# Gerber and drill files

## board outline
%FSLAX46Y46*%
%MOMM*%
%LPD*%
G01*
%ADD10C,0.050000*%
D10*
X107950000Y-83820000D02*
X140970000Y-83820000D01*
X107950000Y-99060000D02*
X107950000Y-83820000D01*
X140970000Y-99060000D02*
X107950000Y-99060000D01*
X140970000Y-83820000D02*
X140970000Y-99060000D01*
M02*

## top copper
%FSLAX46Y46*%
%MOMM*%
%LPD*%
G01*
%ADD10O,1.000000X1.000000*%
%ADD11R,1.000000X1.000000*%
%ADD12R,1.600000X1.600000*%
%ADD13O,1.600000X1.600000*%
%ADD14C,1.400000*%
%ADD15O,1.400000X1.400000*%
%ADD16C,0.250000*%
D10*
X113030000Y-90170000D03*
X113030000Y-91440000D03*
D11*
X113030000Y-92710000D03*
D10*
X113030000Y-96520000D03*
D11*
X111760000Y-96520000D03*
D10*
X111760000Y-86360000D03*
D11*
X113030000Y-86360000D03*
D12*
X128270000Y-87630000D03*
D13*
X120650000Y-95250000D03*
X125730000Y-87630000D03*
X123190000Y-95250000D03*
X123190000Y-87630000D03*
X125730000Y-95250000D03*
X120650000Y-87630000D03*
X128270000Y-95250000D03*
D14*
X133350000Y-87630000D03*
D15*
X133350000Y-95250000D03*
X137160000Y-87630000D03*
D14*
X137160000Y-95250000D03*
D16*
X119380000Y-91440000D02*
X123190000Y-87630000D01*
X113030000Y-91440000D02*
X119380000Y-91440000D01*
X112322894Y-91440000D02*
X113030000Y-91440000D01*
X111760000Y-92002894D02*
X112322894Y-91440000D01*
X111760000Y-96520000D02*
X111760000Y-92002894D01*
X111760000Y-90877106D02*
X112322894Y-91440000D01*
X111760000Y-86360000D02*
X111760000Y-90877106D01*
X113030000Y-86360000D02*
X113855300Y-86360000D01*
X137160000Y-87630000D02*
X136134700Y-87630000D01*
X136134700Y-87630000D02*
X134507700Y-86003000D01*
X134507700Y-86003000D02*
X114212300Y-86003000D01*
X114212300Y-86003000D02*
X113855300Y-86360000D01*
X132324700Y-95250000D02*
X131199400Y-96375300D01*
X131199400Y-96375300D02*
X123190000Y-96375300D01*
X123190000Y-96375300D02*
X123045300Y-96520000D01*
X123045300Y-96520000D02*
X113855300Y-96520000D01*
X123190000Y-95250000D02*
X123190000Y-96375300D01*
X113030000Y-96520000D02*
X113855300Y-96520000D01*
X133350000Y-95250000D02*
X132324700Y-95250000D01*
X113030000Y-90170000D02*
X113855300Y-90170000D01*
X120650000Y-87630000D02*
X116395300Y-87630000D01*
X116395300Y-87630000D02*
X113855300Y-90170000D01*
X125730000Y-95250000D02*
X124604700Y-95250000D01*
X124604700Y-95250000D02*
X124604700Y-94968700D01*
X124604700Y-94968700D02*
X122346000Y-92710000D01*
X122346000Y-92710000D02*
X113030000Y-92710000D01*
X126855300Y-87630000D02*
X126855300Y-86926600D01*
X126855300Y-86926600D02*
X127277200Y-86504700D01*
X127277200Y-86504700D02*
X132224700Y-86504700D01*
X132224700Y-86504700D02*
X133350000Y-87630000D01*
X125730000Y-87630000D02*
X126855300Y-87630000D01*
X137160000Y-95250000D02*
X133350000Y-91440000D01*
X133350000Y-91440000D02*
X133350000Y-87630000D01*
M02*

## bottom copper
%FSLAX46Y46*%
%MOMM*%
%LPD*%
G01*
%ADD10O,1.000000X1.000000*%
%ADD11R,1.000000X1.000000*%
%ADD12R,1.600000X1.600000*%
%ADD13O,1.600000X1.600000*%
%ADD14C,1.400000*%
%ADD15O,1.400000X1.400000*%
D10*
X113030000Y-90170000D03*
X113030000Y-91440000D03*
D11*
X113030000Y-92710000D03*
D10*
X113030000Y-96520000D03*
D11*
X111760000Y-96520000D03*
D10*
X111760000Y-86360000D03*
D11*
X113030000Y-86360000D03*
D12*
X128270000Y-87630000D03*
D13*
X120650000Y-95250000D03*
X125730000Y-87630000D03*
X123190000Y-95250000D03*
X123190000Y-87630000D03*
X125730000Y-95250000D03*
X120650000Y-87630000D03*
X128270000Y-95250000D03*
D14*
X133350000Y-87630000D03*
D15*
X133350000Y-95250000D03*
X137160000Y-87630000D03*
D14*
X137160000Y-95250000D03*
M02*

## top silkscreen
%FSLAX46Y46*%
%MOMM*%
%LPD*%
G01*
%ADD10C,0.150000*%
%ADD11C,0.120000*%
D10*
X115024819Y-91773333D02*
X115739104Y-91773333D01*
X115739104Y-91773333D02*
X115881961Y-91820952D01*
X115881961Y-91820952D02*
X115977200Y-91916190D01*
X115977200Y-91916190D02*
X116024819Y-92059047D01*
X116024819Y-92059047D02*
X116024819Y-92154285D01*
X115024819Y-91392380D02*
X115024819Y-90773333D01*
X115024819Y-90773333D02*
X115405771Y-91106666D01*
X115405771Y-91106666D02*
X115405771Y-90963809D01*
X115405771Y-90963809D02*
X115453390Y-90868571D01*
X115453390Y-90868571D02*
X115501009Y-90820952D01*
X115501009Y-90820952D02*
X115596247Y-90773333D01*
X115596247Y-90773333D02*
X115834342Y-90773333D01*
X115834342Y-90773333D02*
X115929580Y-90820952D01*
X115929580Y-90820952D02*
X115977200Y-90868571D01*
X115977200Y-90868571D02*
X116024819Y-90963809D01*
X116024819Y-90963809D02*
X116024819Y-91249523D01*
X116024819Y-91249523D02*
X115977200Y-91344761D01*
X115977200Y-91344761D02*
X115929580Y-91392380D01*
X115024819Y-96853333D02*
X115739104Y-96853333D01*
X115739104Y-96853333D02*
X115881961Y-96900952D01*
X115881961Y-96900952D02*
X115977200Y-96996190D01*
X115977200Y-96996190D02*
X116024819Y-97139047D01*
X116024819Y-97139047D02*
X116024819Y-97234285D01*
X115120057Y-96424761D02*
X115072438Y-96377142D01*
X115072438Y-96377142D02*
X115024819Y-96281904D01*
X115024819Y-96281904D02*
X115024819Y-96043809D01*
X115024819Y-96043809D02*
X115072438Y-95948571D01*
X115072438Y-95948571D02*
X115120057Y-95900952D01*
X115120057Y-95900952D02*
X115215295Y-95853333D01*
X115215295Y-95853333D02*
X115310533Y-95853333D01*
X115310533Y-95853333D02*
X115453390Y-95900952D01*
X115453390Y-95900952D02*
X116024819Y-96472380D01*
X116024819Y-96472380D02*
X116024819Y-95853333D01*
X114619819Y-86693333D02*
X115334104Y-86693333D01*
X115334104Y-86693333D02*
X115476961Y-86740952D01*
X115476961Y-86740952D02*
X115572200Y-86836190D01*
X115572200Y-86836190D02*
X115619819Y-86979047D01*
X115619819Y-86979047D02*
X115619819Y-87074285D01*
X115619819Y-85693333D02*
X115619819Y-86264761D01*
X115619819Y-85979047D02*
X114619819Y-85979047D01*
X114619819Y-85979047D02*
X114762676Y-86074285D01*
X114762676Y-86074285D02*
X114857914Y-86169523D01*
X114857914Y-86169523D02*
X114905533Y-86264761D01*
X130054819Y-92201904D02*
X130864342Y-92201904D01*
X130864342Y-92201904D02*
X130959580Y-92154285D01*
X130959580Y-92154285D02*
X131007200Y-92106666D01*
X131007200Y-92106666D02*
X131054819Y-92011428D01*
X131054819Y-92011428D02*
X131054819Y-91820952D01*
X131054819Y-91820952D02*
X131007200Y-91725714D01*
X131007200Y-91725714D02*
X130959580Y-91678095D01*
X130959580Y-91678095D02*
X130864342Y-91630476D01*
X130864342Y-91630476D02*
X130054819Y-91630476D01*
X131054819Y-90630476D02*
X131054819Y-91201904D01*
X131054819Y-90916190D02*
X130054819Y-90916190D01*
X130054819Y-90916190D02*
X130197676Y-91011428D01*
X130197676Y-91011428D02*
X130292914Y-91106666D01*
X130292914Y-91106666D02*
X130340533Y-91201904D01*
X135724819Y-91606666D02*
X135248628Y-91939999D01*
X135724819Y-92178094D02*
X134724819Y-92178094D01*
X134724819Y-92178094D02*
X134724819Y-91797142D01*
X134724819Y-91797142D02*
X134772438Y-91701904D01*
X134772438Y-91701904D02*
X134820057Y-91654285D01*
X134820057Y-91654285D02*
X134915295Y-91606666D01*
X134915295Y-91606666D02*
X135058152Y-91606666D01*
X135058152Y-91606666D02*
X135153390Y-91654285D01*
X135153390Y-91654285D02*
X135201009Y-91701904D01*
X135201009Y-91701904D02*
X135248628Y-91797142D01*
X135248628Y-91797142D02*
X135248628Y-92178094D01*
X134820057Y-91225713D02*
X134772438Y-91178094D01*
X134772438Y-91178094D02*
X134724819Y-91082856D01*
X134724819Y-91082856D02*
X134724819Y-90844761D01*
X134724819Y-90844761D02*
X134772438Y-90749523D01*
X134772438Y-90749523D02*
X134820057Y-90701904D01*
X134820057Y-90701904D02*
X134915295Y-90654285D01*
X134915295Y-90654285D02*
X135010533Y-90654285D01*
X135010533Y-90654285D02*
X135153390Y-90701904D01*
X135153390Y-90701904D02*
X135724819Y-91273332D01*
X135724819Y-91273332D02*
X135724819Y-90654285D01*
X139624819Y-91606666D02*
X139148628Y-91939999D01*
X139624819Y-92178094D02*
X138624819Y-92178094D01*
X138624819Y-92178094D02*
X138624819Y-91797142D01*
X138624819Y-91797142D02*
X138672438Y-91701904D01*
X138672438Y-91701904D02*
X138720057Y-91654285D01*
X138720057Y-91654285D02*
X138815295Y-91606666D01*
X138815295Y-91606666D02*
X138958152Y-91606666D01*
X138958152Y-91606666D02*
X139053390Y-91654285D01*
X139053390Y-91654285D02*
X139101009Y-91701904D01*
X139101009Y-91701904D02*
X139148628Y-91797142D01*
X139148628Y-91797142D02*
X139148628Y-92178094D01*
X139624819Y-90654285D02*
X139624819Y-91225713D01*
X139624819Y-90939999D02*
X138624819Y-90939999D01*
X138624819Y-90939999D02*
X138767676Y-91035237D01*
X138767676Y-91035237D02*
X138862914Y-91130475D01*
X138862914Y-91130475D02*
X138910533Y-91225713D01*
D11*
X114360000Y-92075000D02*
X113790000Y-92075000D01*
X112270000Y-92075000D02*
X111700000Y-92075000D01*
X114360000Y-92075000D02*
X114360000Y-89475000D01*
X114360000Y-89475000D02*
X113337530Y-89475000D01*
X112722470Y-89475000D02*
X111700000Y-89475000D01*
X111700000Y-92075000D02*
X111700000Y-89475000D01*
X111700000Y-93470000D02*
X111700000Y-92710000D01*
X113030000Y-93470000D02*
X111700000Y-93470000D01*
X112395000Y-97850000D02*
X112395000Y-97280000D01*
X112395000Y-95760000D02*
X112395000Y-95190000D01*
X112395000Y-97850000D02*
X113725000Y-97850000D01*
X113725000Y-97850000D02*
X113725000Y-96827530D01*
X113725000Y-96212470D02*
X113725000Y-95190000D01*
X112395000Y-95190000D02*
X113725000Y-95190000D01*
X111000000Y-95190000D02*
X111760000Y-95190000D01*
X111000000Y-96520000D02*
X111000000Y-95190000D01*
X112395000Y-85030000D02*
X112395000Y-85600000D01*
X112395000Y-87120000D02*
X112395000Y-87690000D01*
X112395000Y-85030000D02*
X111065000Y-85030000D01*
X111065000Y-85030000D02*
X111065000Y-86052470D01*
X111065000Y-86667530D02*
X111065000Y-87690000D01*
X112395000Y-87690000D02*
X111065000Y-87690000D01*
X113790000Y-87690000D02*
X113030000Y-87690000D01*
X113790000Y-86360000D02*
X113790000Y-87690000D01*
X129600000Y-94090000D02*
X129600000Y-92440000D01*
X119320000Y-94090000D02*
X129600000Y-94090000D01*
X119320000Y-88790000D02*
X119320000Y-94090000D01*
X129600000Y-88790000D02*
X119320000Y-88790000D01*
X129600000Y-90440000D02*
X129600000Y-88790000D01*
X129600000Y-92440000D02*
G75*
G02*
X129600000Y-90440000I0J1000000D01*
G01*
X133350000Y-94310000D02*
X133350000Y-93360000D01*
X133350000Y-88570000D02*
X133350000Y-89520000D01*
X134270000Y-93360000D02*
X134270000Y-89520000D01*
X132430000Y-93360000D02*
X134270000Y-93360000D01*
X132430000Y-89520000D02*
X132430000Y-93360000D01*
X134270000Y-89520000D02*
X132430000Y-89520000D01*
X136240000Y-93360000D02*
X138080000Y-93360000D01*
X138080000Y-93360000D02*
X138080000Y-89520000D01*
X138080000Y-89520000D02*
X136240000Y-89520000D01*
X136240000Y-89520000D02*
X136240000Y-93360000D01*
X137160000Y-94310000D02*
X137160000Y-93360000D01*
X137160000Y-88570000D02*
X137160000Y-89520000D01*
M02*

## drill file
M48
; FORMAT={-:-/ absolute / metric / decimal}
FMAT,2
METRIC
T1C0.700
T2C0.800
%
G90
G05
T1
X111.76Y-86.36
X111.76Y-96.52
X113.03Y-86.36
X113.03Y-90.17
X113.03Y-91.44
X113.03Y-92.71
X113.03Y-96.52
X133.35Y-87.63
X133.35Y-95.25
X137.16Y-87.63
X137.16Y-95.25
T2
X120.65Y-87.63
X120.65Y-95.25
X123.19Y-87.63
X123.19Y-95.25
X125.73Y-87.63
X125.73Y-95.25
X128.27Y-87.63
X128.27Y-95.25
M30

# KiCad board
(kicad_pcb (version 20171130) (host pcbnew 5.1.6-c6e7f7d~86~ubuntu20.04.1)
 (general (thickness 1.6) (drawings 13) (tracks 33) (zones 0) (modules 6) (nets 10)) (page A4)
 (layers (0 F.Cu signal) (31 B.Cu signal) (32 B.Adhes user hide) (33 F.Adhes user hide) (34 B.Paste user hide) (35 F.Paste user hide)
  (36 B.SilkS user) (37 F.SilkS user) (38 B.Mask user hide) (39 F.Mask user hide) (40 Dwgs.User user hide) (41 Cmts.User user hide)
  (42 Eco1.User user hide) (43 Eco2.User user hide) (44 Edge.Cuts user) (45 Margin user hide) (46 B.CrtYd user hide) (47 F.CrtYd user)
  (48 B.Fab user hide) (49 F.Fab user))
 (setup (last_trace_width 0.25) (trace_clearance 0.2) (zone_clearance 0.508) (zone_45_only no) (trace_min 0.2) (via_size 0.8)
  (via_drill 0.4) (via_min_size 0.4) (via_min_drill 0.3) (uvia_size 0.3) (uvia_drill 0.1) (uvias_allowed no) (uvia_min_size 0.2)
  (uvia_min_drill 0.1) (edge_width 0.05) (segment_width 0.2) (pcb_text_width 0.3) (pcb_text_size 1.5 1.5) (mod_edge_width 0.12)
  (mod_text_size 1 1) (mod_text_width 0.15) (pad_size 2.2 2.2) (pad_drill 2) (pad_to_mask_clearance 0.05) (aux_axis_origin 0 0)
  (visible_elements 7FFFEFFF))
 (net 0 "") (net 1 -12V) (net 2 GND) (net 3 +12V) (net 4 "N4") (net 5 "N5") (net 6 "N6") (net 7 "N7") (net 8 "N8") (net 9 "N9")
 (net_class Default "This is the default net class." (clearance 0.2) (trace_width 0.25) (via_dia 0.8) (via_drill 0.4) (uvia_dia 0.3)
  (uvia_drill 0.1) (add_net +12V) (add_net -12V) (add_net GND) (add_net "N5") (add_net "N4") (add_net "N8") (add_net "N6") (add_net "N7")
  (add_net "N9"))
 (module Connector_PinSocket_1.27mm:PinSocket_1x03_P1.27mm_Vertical (layer F.Cu) (at 113.03 92.71 180)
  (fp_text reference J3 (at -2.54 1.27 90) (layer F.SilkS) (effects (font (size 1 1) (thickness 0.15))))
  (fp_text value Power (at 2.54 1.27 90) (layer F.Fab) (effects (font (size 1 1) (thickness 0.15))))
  (fp_line (start -1.33 0.635) (end -0.76 0.635) (layer F.SilkS) (width 0.12))
  (fp_line (start 0.76 0.635) (end 1.33 0.635) (layer F.SilkS) (width 0.12))
  (fp_line (start -1.33 0.635) (end -1.33 3.235) (layer F.SilkS) (width 0.12))
  (fp_line (start -1.33 3.235) (end -0.30753 3.235) (layer F.SilkS) (width 0.12))
  (fp_line (start 0.30753 3.235) (end 1.33 3.235) (layer F.SilkS) (width 0.12))
  (fp_line (start 1.33 0.635) (end 1.33 3.235) (layer F.SilkS) (width 0.12))
  (fp_line (start 1.33 -0.76) (end 1.33 0) (layer F.SilkS) (width 0.12))
  (fp_line (start 0 -0.76) (end 1.33 -0.76) (layer F.SilkS) (width 0.12))
  (pad 3 thru_hole oval (at 0 2.54 180) (size 1 1) (drill 0.7) (layers *.Cu *.Mask) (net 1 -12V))
  (pad 2 thru_hole oval (at 0 1.27 180) (size 1 1) (drill 0.7) (layers *.Cu *.Mask) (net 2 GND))
  (pad 1 thru_hole rect (at 0 0 180) (size 1 1) (drill 0.7) (layers *.Cu *.Mask) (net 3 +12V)))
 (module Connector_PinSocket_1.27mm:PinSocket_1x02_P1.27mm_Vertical (layer F.Cu) (at 111.76 96.52 90)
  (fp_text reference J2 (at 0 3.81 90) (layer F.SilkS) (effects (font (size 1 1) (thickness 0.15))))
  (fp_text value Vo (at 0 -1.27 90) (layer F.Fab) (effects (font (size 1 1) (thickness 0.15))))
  (fp_line (start -1.33 0.635) (end -0.76 0.635) (layer F.SilkS) (width 0.12))
  (fp_line (start 0.76 0.635) (end 1.33 0.635) (layer F.SilkS) (width 0.12))
  (fp_line (start -1.33 0.635) (end -1.33 1.965) (layer F.SilkS) (width 0.12))
  (fp_line (start -1.33 1.965) (end -0.30753 1.965) (layer F.SilkS) (width 0.12))
  (fp_line (start 0.30753 1.965) (end 1.33 1.965) (layer F.SilkS) (width 0.12))
  (fp_line (start 1.33 0.635) (end 1.33 1.965) (layer F.SilkS) (width 0.12))
  (fp_line (start 1.33 -0.76) (end 1.33 0) (layer F.SilkS) (width 0.12))
  (fp_line (start 0 -0.76) (end 1.33 -0.76) (layer F.SilkS) (width 0.12))
  (pad 2 thru_hole oval (at 0 1.27 90) (size 1 1) (drill 0.7) (layers *.Cu *.Mask) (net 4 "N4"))
  (pad 1 thru_hole rect (at 0 0 90) (size 1 1) (drill 0.7) (layers *.Cu *.Mask) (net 2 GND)))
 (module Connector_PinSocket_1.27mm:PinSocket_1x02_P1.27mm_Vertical (layer F.Cu) (at 113.03 86.36 270)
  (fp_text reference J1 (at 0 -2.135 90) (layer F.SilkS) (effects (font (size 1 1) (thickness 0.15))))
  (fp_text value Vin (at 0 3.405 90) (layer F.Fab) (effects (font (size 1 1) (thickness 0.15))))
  (fp_line (start -1.33 0.635) (end -0.76 0.635) (layer F.SilkS) (width 0.12))
  (fp_line (start 0.76 0.635) (end 1.33 0.635) (layer F.SilkS) (width 0.12))
  (fp_line (start -1.33 0.635) (end -1.33 1.965) (layer F.SilkS) (width 0.12))
  (fp_line (start -1.33 1.965) (end -0.30753 1.965) (layer F.SilkS) (width 0.12))
  (fp_line (start 0.30753 1.965) (end 1.33 1.965) (layer F.SilkS) (width 0.12))
  (fp_line (start 1.33 0.635) (end 1.33 1.965) (layer F.SilkS) (width 0.12))
  (fp_line (start 1.33 -0.76) (end 1.33 0) (layer F.SilkS) (width 0.12))
  (fp_line (start 0 -0.76) (end 1.33 -0.76) (layer F.SilkS) (width 0.12))
  (pad 2 thru_hole oval (at 0 1.27 270) (size 1 1) (drill 0.7) (layers *.Cu *.Mask) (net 2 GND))
  (pad 1 thru_hole rect (at 0 0 270) (size 1 1) (drill 0.7) (layers *.Cu *.Mask) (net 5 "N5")))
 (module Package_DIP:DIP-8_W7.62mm (layer F.Cu) (at 128.27 87.63 270)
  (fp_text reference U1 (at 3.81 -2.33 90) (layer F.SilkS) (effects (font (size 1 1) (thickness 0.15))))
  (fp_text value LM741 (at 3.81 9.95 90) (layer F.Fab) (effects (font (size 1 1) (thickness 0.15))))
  (fp_line (start 6.46 -1.33) (end 4.81 -1.33) (layer F.SilkS) (width 0.12))
  (fp_line (start 6.46 8.95) (end 6.46 -1.33) (layer F.SilkS) (width 0.12))
  (fp_line (start 1.16 8.95) (end 6.46 8.95) (layer F.SilkS) (width 0.12))
  (fp_line (start 1.16 -1.33) (end 1.16 8.95) (layer F.SilkS) (width 0.12))
  (fp_line (start 2.81 -1.33) (end 1.16 -1.33) (layer F.SilkS) (width 0.12))
  (fp_arc (start 3.81 -1.33) (end 2.81 -1.33) (angle -180) (layer F.SilkS) (width 0.12))
  (pad 1 thru_hole rect (at 0 0 270) (size 1.6 1.6) (drill 0.8) (layers *.Cu *.Mask) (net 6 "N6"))
  (pad 5 thru_hole oval (at 7.62 7.62 270) (size 1.6 1.6) (drill 0.8) (layers *.Cu *.Mask) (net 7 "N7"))
  (pad 2 thru_hole oval (at 0 2.54 270) (size 1.6 1.6) (drill 0.8) (layers *.Cu *.Mask) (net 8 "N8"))
  (pad 6 thru_hole oval (at 7.62 5.08 270) (size 1.6 1.6) (drill 0.8) (layers *.Cu *.Mask) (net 4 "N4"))
  (pad 3 thru_hole oval (at 0 5.08 270) (size 1.6 1.6) (drill 0.8) (layers *.Cu *.Mask) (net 2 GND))
  (pad 7 thru_hole oval (at 7.62 2.54 270) (size 1.6 1.6) (drill 0.8) (layers *.Cu *.Mask) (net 3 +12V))
  (pad 4 thru_hole oval (at 0 7.62 270) (size 1.6 1.6) (drill 0.8) (layers *.Cu *.Mask) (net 1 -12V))
  (pad 8 thru_hole oval (at 7.62 0 270) (size 1.6 1.6) (drill 0.8) (layers *.Cu *.Mask) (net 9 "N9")))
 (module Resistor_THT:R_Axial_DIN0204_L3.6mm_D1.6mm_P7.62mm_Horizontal (layer F.Cu) (at 133.35 87.63 270)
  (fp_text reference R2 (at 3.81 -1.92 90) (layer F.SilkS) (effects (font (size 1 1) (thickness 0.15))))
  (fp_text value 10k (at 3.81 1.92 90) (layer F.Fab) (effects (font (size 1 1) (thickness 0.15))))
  (fp_line (start 6.68 0) (end 5.73 0) (layer F.SilkS) (width 0.12))
  (fp_line (start 0.94 0) (end 1.89 0) (layer F.SilkS) (width 0.12))
  (fp_line (start 5.73 -0.92) (end 1.89 -0.92) (layer F.SilkS) (width 0.12))
  (fp_line (start 5.73 0.92) (end 5.73 -0.92) (layer F.SilkS) (width 0.12))
  (fp_line (start 1.89 0.92) (end 5.73 0.92) (layer F.SilkS) (width 0.12))
  (fp_line (start 1.89 -0.92) (end 1.89 0.92) (layer F.SilkS) (width 0.12))
  (pad 1 thru_hole circle (at 0 0 270) (size 1.4 1.4) (drill 0.7) (layers *.Cu *.Mask) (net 8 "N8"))
  (pad 2 thru_hole oval (at 7.62 0 270) (size 1.4 1.4) (drill 0.7) (layers *.Cu *.Mask) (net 4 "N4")))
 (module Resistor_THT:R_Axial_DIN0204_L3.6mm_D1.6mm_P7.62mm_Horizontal (layer F.Cu) (at 137.16 95.25 90)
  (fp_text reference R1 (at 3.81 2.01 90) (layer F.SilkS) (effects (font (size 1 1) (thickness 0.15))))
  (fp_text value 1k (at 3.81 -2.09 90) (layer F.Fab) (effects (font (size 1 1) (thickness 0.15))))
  (fp_line (start 1.89 -0.92) (end 1.89 0.92) (layer F.SilkS) (width 0.12))
  (fp_line (start 1.89 0.92) (end 5.73 0.92) (layer F.SilkS) (width 0.12))
  (fp_line (start 5.73 0.92) (end 5.73 -0.92) (layer F.SilkS) (width 0.12))
  (fp_line (start 5.73 -0.92) (end 1.89 -0.92) (layer F.SilkS) (width 0.12))
  (fp_line (start 0.94 0) (end 1.89 0) (layer F.SilkS) (width 0.12))
  (fp_line (start 6.68 0) (end 5.73 0) (layer F.SilkS) (width 0.12))
  (pad 2 thru_hole oval (at 7.62 0 90) (size 1.4 1.4) (drill 0.7) (layers *.Cu *.Mask) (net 5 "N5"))
  (pad 1 thru_hole circle (at 0 0 90) (size 1.4 1.4) (drill 0.7) (layers *.Cu *.Mask) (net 8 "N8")))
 (gr_line (start 107.95 83.82) (end 140.97 83.82) (layer Edge.Cuts) (width 0.05))
 (gr_line (start 107.95 99.06) (end 107.95 83.82) (layer Edge.Cuts) (width 0.05))
 (gr_line (start 140.97 99.06) (end 107.95 99.06) (layer Edge.Cuts) (width 0.05))
 (gr_line (start 140.97 83.82) (end 140.97 99.06) (layer Edge.Cuts) (width 0.05))
 (segment (start 119.38 91.44) (end 123.19 87.63) (width 0.25) (layer F.Cu) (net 2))
 (segment (start 113.03 91.44) (end 119.38 91.44) (width 0.25) (layer F.Cu) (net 2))
 (segment (start 112.322894 91.44) (end 113.03 91.44) (width 0.25) (layer F.Cu) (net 2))
 (segment (start 111.76 92.002894) (end 112.322894 91.44) (width 0.25) (layer F.Cu) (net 2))
 (segment (start 111.76 96.52) (end 111.76 92.002894) (width 0.25) (layer F.Cu) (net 2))
 (segment (start 111.76 90.877106) (end 112.322894 91.44) (width 0.25) (layer F.Cu) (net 2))
 (segment (start 111.76 86.36) (end 111.76 90.877106) (width 0.25) (layer F.Cu) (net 2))
 (segment (start 113.03 86.36) (end 113.8553 86.36) (width 0.25) (layer F.Cu) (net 5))
 (segment (start 137.16 87.63) (end 136.1347 87.63) (width 0.25) (layer F.Cu) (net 5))
 (segment (start 136.1347 87.63) (end 134.5077 86.003) (width 0.25) (layer F.Cu) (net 5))
 (segment (start 134.5077 86.003) (end 114.2123 86.003) (width 0.25) (layer F.Cu) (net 5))
 (segment (start 114.2123 86.003) (end 113.8553 86.36) (width 0.25) (layer F.Cu) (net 5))
 (segment (start 132.3247 95.25) (end 131.1994 96.3753) (width 0.25) (layer F.Cu) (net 4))
 (segment (start 131.1994 96.3753) (end 123.19 96.3753) (width 0.25) (layer F.Cu) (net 4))
 (segment (start 123.19 96.3753) (end 123.0453 96.52) (width 0.25) (layer F.Cu) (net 4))
 (segment (start 123.0453 96.52) (end 113.8553 96.52) (width 0.25) (layer F.Cu) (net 4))
 (segment (start 123.19 95.25) (end 123.19 96.3753) (width 0.25) (layer F.Cu) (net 4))
 (segment (start 113.03 96.52) (end 113.8553 96.52) (width 0.25) (layer F.Cu) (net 4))
 (segment (start 133.35 95.25) (end 132.3247 95.25) (width 0.25) (layer F.Cu) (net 4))
 (segment (start 113.03 90.17) (end 113.8553 90.17) (width 0.25) (layer F.Cu) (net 1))
 (segment (start 120.65 87.63) (end 116.3953 87.63) (width 0.25) (layer F.Cu) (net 1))
 (segment (start 116.3953 87.63) (end 113.8553 90.17) (width 0.25) (layer F.Cu) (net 1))
 (segment (start 125.73 95.25) (end 124.6047 95.25) (width 0.25) (layer F.Cu) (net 3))
 (segment (start 124.6047 95.25) (end 124.6047 94.9687) (width 0.25) (layer F.Cu) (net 3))
 (segment (start 124.6047 94.9687) (end 122.346 92.71) (width 0.25) (layer F.Cu) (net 3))
 (segment (start 122.346 92.71) (end 113.03 92.71) (width 0.25) (layer F.Cu) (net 3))
 (segment (start 126.8553 87.63) (end 126.8553 86.9266) (width 0.25) (layer F.Cu) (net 8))
 (segment (start 126.8553 86.9266) (end 127.2772 86.5047) (width 0.25) (layer F.Cu) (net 8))
 (segment (start 127.2772 86.5047) (end 132.2247 86.5047) (width 0.25) (layer F.Cu) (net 8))
 (segment (start 132.2247 86.5047) (end 133.35 87.63) (width 0.25) (layer F.Cu) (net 8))
 (segment (start 125.73 87.63) (end 126.8553 87.63) (width 0.25) (layer F.Cu) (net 8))
 (segment (start 137.16 95.25) (end 133.35 91.44) (width 0.25) (layer F.Cu) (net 8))
 (segment (start 133.35 91.44) (end 133.35 87.63) (width 0.25) (layer F.Cu) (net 8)))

